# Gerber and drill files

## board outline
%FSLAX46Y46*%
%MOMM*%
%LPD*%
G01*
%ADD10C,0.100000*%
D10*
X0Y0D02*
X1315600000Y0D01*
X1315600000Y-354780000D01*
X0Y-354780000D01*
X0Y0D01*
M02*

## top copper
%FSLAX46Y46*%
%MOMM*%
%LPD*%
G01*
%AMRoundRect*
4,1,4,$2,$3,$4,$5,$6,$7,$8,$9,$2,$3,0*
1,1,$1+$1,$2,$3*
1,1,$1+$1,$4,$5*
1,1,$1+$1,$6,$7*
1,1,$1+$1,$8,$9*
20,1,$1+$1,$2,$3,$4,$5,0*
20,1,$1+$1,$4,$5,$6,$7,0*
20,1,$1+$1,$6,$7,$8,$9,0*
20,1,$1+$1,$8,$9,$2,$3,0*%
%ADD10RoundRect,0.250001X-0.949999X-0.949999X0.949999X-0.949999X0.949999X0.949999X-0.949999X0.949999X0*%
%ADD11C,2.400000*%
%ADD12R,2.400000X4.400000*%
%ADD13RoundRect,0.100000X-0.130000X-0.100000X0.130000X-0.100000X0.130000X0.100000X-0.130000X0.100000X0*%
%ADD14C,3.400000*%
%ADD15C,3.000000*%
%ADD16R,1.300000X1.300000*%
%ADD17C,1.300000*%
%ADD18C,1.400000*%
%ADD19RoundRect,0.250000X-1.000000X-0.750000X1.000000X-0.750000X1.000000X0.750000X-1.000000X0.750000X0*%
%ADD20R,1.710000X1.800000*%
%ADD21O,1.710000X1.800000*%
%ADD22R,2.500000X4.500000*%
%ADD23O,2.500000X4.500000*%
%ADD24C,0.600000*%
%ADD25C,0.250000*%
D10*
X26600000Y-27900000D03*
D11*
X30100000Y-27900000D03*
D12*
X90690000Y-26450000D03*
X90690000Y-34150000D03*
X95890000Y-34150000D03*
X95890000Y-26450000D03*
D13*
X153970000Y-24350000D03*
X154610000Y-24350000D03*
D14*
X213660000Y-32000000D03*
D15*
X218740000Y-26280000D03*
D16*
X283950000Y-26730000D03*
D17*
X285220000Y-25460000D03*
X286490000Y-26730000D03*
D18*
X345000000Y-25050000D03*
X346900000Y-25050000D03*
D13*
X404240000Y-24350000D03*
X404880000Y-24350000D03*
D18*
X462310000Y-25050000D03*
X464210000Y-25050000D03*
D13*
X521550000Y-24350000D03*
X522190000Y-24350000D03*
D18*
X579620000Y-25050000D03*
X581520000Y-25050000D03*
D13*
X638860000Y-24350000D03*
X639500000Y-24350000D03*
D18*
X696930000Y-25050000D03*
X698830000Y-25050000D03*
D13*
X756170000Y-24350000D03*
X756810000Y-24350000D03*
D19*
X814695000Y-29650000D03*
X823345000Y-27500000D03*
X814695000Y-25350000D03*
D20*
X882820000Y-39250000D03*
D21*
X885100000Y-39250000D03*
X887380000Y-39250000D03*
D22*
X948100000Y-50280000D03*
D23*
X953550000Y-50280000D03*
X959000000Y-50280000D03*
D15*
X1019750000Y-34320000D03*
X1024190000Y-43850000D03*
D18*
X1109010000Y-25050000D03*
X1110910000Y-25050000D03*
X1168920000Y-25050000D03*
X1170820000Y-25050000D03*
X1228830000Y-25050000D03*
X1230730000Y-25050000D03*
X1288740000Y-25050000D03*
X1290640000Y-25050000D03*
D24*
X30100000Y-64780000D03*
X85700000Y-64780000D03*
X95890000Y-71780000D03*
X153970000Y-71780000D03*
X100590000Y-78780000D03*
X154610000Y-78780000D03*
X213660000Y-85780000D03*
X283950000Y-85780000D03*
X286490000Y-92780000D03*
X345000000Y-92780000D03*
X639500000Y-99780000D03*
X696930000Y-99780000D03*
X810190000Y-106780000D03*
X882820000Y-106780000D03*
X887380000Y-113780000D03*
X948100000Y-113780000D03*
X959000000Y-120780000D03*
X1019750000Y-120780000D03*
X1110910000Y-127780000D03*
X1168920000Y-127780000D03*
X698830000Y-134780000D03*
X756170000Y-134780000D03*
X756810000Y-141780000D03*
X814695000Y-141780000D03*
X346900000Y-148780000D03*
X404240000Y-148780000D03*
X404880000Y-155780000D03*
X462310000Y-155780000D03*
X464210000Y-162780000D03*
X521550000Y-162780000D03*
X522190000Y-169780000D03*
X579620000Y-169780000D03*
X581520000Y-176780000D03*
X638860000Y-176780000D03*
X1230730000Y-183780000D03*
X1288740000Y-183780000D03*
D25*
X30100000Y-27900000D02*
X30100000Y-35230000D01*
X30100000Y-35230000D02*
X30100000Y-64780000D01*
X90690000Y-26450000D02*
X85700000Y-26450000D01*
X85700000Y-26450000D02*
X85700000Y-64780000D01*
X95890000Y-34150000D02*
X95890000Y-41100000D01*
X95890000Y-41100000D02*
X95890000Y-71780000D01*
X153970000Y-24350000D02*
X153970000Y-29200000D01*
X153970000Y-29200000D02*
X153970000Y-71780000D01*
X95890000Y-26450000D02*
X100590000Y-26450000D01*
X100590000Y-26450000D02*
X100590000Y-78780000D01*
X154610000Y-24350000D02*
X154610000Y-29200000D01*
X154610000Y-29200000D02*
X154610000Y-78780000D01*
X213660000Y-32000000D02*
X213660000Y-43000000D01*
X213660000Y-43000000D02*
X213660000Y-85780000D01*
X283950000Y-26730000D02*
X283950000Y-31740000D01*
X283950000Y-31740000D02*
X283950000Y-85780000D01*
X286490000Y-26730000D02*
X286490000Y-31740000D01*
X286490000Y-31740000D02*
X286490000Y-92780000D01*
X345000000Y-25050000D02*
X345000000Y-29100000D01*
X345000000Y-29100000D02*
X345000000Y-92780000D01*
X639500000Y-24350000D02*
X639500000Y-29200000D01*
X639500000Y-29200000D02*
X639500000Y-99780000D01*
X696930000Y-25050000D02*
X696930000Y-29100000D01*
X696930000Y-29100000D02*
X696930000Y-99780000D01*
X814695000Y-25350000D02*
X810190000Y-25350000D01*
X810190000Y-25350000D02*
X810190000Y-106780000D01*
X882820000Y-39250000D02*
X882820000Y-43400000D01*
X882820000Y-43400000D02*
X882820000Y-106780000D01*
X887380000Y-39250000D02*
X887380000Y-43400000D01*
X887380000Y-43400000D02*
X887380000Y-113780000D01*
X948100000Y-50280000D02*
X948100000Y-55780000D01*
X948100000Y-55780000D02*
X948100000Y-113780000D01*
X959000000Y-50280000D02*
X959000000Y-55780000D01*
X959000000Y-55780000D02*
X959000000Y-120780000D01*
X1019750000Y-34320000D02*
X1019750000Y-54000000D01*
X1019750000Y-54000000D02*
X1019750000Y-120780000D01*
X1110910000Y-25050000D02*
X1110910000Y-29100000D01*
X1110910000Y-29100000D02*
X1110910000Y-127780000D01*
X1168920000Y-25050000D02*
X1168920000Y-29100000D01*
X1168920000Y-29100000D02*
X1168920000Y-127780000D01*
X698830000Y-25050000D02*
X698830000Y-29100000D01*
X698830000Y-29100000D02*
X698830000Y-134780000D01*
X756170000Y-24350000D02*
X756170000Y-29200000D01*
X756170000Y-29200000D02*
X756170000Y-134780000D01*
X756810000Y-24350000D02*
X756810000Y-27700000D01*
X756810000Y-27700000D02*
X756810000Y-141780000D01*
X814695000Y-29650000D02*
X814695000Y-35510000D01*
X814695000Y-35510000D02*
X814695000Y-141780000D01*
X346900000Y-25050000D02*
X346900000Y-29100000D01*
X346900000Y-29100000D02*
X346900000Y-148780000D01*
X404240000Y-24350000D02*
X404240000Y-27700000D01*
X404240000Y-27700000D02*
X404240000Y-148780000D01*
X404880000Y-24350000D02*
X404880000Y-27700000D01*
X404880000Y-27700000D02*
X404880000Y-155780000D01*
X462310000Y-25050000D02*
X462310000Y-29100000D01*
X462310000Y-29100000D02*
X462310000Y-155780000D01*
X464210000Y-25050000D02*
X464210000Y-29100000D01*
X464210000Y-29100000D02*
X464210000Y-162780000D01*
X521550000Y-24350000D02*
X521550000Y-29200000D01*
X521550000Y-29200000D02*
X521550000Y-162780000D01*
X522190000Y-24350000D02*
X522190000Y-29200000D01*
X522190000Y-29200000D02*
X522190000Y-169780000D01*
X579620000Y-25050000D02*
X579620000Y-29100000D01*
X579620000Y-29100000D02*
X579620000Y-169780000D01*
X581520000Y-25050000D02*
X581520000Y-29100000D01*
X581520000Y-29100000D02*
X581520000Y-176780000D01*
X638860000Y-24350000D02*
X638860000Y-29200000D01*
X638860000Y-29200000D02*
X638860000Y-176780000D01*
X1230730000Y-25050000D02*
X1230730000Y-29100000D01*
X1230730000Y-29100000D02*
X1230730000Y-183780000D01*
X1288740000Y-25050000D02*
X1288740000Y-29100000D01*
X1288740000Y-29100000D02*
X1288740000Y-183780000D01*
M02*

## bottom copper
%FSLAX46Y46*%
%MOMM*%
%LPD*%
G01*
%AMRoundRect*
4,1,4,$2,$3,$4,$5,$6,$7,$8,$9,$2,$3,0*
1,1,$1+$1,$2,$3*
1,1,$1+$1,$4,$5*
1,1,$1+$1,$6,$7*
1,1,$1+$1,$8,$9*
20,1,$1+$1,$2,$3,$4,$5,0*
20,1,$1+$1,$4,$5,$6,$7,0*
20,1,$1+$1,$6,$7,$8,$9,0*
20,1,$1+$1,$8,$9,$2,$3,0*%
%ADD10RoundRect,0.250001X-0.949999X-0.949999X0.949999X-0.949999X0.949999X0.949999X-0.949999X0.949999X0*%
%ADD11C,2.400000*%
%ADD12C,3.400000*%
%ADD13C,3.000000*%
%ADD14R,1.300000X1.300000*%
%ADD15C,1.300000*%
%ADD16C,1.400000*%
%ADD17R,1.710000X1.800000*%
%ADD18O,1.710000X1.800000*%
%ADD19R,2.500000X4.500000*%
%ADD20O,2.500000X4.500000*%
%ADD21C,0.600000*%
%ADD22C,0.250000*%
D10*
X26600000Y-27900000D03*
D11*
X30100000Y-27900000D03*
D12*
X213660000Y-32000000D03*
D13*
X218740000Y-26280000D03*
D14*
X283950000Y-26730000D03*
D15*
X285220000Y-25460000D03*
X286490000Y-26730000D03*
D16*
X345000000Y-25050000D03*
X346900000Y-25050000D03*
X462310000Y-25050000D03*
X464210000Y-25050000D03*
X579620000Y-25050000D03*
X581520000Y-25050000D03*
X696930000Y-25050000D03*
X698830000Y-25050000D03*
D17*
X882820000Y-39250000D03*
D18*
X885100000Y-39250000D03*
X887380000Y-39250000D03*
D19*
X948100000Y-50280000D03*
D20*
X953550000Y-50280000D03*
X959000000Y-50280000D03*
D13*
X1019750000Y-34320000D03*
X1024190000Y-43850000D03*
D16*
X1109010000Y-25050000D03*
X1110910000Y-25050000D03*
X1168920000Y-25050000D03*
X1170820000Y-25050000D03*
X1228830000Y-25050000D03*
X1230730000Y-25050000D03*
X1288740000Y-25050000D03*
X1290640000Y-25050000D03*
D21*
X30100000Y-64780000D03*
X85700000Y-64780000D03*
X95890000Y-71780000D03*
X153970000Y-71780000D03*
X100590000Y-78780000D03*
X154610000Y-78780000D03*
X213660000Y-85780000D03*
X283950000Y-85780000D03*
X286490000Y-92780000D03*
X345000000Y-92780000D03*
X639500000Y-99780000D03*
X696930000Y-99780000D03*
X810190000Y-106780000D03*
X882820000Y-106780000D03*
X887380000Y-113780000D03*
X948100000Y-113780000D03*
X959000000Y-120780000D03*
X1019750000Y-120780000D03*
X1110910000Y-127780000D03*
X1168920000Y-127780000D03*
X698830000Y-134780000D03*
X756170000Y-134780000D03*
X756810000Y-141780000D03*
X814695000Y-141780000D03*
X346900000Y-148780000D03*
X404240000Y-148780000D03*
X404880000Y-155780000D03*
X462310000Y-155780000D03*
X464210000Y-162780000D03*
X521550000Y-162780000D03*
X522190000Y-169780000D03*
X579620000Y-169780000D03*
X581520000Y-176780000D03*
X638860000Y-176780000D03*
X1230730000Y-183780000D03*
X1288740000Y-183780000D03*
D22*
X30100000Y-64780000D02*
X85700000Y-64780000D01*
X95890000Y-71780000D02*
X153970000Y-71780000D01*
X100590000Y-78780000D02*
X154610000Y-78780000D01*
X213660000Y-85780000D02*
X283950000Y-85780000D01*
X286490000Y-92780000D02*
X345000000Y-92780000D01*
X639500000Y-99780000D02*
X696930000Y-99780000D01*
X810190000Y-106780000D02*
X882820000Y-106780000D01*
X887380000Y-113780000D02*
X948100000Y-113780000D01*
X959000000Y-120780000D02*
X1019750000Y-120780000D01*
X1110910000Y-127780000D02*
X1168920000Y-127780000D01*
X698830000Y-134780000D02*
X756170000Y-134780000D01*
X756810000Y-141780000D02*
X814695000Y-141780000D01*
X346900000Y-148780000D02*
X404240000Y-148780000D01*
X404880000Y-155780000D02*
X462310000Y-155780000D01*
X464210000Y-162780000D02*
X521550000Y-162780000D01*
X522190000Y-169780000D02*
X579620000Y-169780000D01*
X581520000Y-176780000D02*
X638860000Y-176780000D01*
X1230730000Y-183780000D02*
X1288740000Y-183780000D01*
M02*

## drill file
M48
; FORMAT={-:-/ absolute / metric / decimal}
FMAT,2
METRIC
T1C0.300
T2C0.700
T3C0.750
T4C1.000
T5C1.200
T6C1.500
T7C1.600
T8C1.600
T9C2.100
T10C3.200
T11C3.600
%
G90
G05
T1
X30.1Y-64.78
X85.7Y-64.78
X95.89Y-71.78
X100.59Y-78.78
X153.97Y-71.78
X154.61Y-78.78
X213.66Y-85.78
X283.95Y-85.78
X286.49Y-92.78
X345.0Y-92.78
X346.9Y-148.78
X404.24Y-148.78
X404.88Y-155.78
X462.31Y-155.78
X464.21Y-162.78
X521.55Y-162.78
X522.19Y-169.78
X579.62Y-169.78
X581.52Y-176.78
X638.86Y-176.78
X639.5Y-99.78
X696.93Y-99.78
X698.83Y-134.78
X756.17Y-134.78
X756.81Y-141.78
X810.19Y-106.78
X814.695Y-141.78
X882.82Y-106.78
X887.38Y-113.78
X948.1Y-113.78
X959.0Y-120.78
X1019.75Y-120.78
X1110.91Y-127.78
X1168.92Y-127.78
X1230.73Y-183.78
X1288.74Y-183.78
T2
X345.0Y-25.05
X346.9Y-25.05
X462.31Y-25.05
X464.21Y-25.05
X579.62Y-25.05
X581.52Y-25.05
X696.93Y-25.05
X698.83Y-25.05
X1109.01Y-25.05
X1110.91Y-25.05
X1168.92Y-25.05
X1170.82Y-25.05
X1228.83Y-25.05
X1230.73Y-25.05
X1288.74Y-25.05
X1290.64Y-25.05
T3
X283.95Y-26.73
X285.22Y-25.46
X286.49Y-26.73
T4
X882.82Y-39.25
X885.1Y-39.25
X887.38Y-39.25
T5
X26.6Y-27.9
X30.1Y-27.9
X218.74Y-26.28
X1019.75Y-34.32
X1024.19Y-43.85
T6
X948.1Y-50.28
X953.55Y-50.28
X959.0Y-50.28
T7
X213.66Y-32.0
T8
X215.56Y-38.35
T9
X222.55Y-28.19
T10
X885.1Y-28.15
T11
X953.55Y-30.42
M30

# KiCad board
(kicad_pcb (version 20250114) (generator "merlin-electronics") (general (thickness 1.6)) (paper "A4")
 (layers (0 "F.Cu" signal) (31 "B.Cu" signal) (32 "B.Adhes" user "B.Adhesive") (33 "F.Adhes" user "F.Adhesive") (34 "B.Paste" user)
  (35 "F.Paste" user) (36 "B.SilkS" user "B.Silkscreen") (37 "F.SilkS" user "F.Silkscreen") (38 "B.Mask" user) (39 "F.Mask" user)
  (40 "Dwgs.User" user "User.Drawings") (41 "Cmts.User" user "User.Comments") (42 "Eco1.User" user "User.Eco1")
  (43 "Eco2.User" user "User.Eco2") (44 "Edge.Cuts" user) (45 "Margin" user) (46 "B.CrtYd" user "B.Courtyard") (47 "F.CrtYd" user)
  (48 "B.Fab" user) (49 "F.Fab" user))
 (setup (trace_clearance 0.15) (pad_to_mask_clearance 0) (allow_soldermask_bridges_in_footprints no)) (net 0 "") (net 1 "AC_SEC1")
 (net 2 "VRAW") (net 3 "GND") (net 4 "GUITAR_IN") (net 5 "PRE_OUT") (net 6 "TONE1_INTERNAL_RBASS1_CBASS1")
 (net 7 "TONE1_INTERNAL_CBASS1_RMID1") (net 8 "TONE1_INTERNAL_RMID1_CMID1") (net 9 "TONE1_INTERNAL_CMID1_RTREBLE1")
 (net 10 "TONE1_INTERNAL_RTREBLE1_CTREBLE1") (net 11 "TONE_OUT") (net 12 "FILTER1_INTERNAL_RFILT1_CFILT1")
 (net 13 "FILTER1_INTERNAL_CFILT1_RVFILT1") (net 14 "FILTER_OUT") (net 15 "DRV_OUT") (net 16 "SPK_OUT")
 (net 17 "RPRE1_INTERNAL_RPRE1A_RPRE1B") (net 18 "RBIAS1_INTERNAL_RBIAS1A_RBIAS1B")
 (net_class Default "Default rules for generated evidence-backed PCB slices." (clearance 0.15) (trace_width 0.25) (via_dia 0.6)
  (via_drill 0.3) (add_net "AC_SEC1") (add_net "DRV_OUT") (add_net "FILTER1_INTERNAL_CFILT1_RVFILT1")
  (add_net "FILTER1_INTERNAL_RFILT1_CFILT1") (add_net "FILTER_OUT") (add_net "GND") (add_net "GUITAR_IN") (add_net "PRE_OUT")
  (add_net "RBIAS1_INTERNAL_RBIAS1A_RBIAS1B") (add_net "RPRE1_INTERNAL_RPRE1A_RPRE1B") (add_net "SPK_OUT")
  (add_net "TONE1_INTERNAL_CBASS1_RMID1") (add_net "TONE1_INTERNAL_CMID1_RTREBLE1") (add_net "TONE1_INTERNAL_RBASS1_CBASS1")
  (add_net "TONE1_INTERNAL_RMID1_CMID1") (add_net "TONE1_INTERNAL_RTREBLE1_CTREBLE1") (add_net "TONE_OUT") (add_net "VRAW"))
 (gr_rect (start 0 0) (end 1315.6 354.78) (stroke (width 0.1) (type default)) (fill no) (layer "Edge.Cuts"))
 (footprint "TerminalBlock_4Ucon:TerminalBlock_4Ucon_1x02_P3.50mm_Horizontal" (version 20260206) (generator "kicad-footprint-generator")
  (layer "F.Cu") (at 26.6 27.9 0)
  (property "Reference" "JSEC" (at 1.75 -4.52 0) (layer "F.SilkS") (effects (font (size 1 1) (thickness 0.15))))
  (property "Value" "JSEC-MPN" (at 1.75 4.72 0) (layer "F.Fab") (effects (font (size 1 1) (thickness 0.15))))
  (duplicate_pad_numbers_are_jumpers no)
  (pad "1" thru_hole roundrect (at 0 0) (size 2.4 2.4) (drill 1.2) (layers "*.Cu" "*.Mask") (remove_unused_layers no)
   (roundrect_rratio 0.104167))
  (pad "2" thru_hole circle (at 3.5 0) (size 2.4 2.4) (drill 1.2) (layers "*.Cu" "*.Mask") (remove_unused_layers no) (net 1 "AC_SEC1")))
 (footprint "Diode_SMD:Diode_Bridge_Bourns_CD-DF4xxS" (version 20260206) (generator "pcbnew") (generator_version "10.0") (layer "F.Cu")
  (at 93.29 30.3 0)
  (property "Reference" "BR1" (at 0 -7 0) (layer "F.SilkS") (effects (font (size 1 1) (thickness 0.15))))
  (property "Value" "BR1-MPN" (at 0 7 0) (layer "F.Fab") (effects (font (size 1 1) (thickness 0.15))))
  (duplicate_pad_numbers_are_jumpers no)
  (pad "1" smd rect (at -2.6 -3.85) (size 2.4 4.4) (layers "F.Cu" "F.Mask" "F.Paste") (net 1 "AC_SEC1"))
  (pad "2" smd rect (at -2.6 3.85) (size 2.4 4.4) (layers "F.Cu" "F.Mask" "F.Paste"))
  (pad "3" smd rect (at 2.6 3.85) (size 2.4 4.4) (layers "F.Cu" "F.Mask" "F.Paste") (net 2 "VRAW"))
  (pad "4" smd rect (at 2.6 -3.85) (size 2.4 4.4) (layers "F.Cu" "F.Mask" "F.Paste") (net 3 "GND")))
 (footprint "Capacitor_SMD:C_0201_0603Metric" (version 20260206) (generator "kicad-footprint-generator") (layer "F.Cu") (at 154.29 24.35 0)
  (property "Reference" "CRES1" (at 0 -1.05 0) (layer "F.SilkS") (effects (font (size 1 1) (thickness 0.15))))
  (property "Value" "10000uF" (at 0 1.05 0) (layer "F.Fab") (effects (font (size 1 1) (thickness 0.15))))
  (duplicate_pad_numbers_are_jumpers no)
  (pad "" smd roundrect (at -0.345 0) (size 0.318 0.36) (layers "F.Paste") (roundrect_rratio 0.25))
  (pad "" smd roundrect (at 0.345 0) (size 0.318 0.36) (layers "F.Paste") (roundrect_rratio 0.25))
  (pad "1" smd roundrect (at -0.32 0) (size 0.46 0.4) (layers "F.Cu" "F.Mask") (roundrect_rratio 0.25) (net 2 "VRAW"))
  (pad "2" smd roundrect (at 0.32 0) (size 0.46 0.4) (layers "F.Cu" "F.Mask") (roundrect_rratio 0.25) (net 3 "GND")))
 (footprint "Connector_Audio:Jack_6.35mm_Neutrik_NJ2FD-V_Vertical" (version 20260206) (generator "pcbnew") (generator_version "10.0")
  (layer "F.Cu") (at 218.74 26.28 0)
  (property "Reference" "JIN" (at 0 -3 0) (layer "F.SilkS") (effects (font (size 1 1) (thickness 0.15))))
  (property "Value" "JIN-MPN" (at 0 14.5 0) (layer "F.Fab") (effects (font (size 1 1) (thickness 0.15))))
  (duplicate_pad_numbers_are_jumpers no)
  (pad "" np_thru_hole circle (at -3.18 12.07 180) (size 1.6 1.6) (drill 1.6) (layers "*.Cu" "*.Mask"))
  (pad "" np_thru_hole circle (at 3.81 1.91 180) (size 2.1 2.1) (drill 2.1) (layers "*.Cu" "*.Mask"))
  (pad "S" thru_hole circle (at -5.08 5.72 180) (size 3.4 3.4) (drill 1.6) (layers "*.Cu" "*.Mask") (remove_unused_layers no)
   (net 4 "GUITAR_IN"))
  (pad "T" thru_hole circle (at 0 0 180) (size 3 3) (drill 1.2) (layers "*.Cu" "*.Mask") (remove_unused_layers no)))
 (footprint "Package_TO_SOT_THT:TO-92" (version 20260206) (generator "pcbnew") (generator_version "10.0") (layer "F.Cu") (at 283.95 26.73 0)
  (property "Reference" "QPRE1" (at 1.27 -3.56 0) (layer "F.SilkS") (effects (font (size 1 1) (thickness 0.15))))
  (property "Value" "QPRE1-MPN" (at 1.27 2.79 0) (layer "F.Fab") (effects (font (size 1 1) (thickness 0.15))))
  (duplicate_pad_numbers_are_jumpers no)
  (pad "1" thru_hole rect (at 0 0) (size 1.3 1.3) (drill 0.75) (layers "*.Cu" "*.Mask") (remove_unused_layers no) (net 4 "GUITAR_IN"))
  (pad "2" thru_hole circle (at 1.27 -1.27) (size 1.3 1.3) (drill 0.75) (layers "*.Cu" "*.Mask") (remove_unused_layers no))
  (pad "3" thru_hole circle (at 2.54 0) (size 1.3 1.3) (drill 0.75) (layers "*.Cu" "*.Mask") (remove_unused_layers no) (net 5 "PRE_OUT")))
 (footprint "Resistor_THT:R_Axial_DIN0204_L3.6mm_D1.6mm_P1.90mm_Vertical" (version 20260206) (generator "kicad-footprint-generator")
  (layer "F.Cu") (at 345 25.05 0)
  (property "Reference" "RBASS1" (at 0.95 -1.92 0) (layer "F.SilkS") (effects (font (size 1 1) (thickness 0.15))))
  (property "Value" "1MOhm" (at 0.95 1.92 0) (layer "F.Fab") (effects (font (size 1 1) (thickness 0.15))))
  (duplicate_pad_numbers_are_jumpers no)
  (pad "1" thru_hole circle (at 0 0) (size 1.4 1.4) (drill 0.7) (layers "*.Cu" "*.Mask") (remove_unused_layers no) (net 5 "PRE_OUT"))
  (pad "2" thru_hole circle (at 1.9 0) (size 1.4 1.4) (drill 0.7) (layers "*.Cu" "*.Mask") (remove_unused_layers no)
   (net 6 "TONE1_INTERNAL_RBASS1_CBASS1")))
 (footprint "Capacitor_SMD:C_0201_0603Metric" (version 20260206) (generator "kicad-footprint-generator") (layer "F.Cu") (at 404.56 24.35 0)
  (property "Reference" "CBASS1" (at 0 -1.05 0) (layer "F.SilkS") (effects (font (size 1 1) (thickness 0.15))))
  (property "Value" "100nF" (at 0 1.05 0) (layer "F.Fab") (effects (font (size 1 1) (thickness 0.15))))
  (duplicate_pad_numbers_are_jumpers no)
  (pad "" smd roundrect (at -0.345 0) (size 0.318 0.36) (layers "F.Paste") (roundrect_rratio 0.25))
  (pad "" smd roundrect (at 0.345 0) (size 0.318 0.36) (layers "F.Paste") (roundrect_rratio 0.25))
  (pad "1" smd roundrect (at -0.32 0) (size 0.46 0.4) (layers "F.Cu" "F.Mask") (roundrect_rratio 0.25)
   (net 6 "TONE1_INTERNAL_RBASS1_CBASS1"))
  (pad "2" smd roundrect (at 0.32 0) (size 0.46 0.4) (layers "F.Cu" "F.Mask") (roundrect_rratio 0.25) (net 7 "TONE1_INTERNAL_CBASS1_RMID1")))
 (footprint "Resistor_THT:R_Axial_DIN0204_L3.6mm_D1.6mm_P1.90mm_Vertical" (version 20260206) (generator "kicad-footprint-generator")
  (layer "F.Cu") (at 462.31 25.05 0)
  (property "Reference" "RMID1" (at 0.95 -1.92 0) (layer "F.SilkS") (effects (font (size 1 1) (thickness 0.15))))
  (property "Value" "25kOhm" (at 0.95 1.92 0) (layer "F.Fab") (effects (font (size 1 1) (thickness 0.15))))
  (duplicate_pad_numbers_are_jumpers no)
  (pad "1" thru_hole circle (at 0 0) (size 1.4 1.4) (drill 0.7) (layers "*.Cu" "*.Mask") (remove_unused_layers no)
   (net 7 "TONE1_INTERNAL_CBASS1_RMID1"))
  (pad "2" thru_hole circle (at 1.9 0) (size 1.4 1.4) (drill 0.7) (layers "*.Cu" "*.Mask") (remove_unused_layers no)
   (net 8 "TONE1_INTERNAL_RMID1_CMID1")))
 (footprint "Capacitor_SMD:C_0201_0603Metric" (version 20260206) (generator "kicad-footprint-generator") (layer "F.Cu") (at 521.87 24.35 0)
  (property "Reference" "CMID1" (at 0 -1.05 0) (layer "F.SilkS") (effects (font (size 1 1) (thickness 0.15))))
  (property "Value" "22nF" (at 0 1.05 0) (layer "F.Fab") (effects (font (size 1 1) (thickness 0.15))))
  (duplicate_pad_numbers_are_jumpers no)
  (pad "" smd roundrect (at -0.345 0) (size 0.318 0.36) (layers "F.Paste") (roundrect_rratio 0.25))
  (pad "" smd roundrect (at 0.345 0) (size 0.318 0.36) (layers "F.Paste") (roundrect_rratio 0.25))
  (pad "1" smd roundrect (at -0.32 0) (size 0.46 0.4) (layers "F.Cu" "F.Mask") (roundrect_rratio 0.25) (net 8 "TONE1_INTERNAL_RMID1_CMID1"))
  (pad "2" smd roundrect (at 0.32 0) (size 0.46 0.4) (layers "F.Cu" "F.Mask") (roundrect_rratio 0.25)
   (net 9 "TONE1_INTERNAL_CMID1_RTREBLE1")))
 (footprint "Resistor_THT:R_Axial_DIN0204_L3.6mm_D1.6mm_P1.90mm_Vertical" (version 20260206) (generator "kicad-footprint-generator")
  (layer "F.Cu") (at 579.62 25.05 0)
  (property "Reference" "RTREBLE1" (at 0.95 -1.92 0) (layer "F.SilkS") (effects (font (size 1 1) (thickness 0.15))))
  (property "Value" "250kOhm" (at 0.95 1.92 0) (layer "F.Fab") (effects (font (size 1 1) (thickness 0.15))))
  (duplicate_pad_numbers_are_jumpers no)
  (pad "1" thru_hole circle (at 0 0) (size 1.4 1.4) (drill 0.7) (layers "*.Cu" "*.Mask") (remove_unused_layers no)
   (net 9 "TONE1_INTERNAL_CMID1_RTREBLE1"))
  (pad "2" thru_hole circle (at 1.9 0) (size 1.4 1.4) (drill 0.7) (layers "*.Cu" "*.Mask") (remove_unused_layers no)
   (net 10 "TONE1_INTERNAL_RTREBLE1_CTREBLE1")))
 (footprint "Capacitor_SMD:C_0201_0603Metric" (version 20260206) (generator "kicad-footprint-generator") (layer "F.Cu") (at 639.18 24.35 0)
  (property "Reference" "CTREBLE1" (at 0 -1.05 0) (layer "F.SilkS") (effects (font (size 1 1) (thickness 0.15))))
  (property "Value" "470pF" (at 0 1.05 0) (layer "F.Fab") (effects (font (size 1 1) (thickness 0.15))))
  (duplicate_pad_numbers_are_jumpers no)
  (pad "" smd roundrect (at -0.345 0) (size 0.318 0.36) (layers "F.Paste") (roundrect_rratio 0.25))
  (pad "" smd roundrect (at 0.345 0) (size 0.318 0.36) (layers "F.Paste") (roundrect_rratio 0.25))
  (pad "1" smd roundrect (at -0.32 0) (size 0.46 0.4) (layers "F.Cu" "F.Mask") (roundrect_rratio 0.25)
   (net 10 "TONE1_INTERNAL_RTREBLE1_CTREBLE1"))
  (pad "2" smd roundrect (at 0.32 0) (size 0.46 0.4) (layers "F.Cu" "F.Mask") (roundrect_rratio 0.25) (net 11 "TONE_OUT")))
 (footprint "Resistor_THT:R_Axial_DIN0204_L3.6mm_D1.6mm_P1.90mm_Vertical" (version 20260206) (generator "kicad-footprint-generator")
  (layer "F.Cu") (at 696.93 25.05 0)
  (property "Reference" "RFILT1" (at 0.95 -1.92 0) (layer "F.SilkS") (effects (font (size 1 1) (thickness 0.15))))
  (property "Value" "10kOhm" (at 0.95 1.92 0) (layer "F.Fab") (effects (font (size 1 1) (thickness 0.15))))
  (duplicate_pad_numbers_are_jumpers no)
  (pad "1" thru_hole circle (at 0 0) (size 1.4 1.4) (drill 0.7) (layers "*.Cu" "*.Mask") (remove_unused_layers no) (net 11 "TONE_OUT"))
  (pad "2" thru_hole circle (at 1.9 0) (size 1.4 1.4) (drill 0.7) (layers "*.Cu" "*.Mask") (remove_unused_layers no)
   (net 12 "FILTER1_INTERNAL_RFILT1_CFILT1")))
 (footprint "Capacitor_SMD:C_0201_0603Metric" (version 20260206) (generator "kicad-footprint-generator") (layer "F.Cu") (at 756.49 24.35 0)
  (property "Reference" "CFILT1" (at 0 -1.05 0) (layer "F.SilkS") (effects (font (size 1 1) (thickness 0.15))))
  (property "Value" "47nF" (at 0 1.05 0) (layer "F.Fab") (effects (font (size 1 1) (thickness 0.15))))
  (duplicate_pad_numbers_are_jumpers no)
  (pad "" smd roundrect (at -0.345 0) (size 0.318 0.36) (layers "F.Paste") (roundrect_rratio 0.25))
  (pad "" smd roundrect (at 0.345 0) (size 0.318 0.36) (layers "F.Paste") (roundrect_rratio 0.25))
  (pad "1" smd roundrect (at -0.32 0) (size 0.46 0.4) (layers "F.Cu" "F.Mask") (roundrect_rratio 0.25)
   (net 12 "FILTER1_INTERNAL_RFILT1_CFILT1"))
  (pad "2" smd roundrect (at 0.32 0) (size 0.46 0.4) (layers "F.Cu" "F.Mask") (roundrect_rratio 0.25)
   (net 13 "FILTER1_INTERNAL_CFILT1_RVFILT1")))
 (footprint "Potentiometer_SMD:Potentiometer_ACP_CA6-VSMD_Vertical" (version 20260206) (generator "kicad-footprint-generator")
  (layer "F.Cu") (at 819.02 27.5 0)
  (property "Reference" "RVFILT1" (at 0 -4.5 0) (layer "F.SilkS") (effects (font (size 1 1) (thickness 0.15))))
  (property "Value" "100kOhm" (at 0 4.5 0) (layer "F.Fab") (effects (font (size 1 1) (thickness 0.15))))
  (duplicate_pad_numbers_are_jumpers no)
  (pad "1" smd roundrect (at -4.325 2.15) (size 2.5 2) (layers "F.Cu" "F.Mask" "F.Paste") (roundrect_rratio 0.125)
   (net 13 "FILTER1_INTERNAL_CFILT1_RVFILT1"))
  (pad "2" smd roundrect (at 4.325 0) (size 2.5 2) (layers "F.Cu" "F.Mask" "F.Paste") (roundrect_rratio 0.125))
  (pad "3" smd roundrect (at -4.325 -2.15) (size 2.5 2) (layers "F.Cu" "F.Mask" "F.Paste") (roundrect_rratio 0.125) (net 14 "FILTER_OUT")))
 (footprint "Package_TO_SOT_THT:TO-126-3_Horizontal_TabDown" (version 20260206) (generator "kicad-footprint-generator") (layer "F.Cu")
  (at 882.82 39.25 0)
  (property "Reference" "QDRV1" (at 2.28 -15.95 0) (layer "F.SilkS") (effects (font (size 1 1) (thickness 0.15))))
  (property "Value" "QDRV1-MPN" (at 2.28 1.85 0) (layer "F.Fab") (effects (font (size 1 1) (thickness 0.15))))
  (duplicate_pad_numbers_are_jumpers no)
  (pad "" np_thru_hole circle (at 2.28 -11.1) (size 3.2 3.2) (drill 3.2) (layers "*.Cu" "*.Mask"))
  (pad "1" thru_hole rect (at 0 0) (size 1.71 1.8) (drill 1) (layers "*.Cu" "*.Mask") (remove_unused_layers no) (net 14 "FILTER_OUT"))
  (pad "2" thru_hole oval (at 2.28 0) (size 1.71 1.8) (drill 1) (layers "*.Cu" "*.Mask") (remove_unused_layers no))
  (pad "3" thru_hole oval (at 4.56 0) (size 1.71 1.8) (drill 1) (layers "*.Cu" "*.Mask") (remove_unused_layers no) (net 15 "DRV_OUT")))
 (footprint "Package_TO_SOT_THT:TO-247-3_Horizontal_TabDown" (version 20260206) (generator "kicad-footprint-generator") (layer "F.Cu")
  (at 948.1 50.28 0)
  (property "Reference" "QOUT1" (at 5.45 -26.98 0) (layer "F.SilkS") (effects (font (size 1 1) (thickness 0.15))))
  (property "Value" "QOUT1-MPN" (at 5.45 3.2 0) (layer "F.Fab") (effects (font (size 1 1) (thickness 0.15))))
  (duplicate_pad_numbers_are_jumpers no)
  (pad "" np_thru_hole circle (at 5.45 -19.86) (size 3.6 3.6) (drill 3.6) (layers "*.Cu" "*.Mask"))
  (pad "1" thru_hole rect (at 0 0) (size 2.5 4.5) (drill 1.5) (layers "*.Cu" "*.Mask") (remove_unused_layers no) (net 15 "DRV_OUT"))
  (pad "2" thru_hole oval (at 5.45 0) (size 2.5 4.5) (drill 1.5) (layers "*.Cu" "*.Mask") (remove_unused_layers no))
  (pad "3" thru_hole oval (at 10.9 0) (size 2.5 4.5) (drill 1.5) (layers "*.Cu" "*.Mask") (remove_unused_layers no) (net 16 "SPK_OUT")))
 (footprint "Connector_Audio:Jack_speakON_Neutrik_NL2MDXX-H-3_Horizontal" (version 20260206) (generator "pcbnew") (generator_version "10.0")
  (layer "F.Cu") (at 1019.75 34.32 0)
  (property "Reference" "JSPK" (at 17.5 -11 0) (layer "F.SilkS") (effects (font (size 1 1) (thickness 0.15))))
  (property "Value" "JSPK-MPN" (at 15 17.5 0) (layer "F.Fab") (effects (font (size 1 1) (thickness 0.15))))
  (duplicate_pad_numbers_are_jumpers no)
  (pad "1+" thru_hole circle (at 0 0) (size 3 3) (drill 1.2) (layers "*.Cu" "*.Mask") (remove_unused_layers no) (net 16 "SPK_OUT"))
  (pad "1-" thru_hole circle (at 4.44 9.53) (size 3 3) (drill 1.2) (layers "*.Cu" "*.Mask") (remove_unused_layers no)))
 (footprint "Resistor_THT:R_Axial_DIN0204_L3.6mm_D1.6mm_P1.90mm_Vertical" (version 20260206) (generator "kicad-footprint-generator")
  (layer "F.Cu") (at 1109.01 25.05 0)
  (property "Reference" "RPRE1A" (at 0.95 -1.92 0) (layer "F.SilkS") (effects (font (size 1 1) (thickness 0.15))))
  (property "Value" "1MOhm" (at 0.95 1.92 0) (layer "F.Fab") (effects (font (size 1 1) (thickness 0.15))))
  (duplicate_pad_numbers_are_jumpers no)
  (pad "1" thru_hole circle (at 0 0) (size 1.4 1.4) (drill 0.7) (layers "*.Cu" "*.Mask") (remove_unused_layers no))
  (pad "2" thru_hole circle (at 1.9 0) (size 1.4 1.4) (drill 0.7) (layers "*.Cu" "*.Mask") (remove_unused_layers no)
   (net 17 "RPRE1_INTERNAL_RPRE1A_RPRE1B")))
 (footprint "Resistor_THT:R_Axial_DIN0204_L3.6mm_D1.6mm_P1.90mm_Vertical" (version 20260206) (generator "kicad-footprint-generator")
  (layer "F.Cu") (at 1168.92 25.05 0)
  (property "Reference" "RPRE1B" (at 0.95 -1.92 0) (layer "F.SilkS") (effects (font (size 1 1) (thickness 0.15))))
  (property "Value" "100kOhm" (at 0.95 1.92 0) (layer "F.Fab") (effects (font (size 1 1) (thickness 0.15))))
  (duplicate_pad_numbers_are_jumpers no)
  (pad "1" thru_hole circle (at 0 0) (size 1.4 1.4) (drill 0.7) (layers "*.Cu" "*.Mask") (remove_unused_layers no)
   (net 17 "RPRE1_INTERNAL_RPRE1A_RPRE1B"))
  (pad "2" thru_hole circle (at 1.9 0) (size 1.4 1.4) (drill 0.7) (layers "*.Cu" "*.Mask") (remove_unused_layers no)))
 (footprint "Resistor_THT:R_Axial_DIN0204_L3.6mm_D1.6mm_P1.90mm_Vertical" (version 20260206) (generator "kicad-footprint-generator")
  (layer "F.Cu") (at 1228.83 25.05 0)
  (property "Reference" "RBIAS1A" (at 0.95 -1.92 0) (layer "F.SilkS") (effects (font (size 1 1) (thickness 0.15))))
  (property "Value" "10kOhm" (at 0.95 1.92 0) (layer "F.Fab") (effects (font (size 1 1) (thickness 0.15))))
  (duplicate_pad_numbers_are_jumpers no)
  (pad "1" thru_hole circle (at 0 0) (size 1.4 1.4) (drill 0.7) (layers "*.Cu" "*.Mask") (remove_unused_layers no))
  (pad "2" thru_hole circle (at 1.9 0) (size 1.4 1.4) (drill 0.7) (layers "*.Cu" "*.Mask") (remove_unused_layers no)
   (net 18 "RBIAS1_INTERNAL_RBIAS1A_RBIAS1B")))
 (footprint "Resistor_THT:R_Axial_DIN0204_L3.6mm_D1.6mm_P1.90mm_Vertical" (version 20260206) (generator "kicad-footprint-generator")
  (layer "F.Cu") (at 1288.74 25.05 0)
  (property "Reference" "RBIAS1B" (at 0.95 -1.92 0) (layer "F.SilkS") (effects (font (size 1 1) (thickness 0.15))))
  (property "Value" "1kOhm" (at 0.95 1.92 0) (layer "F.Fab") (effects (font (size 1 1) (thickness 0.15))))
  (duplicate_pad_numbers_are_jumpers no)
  (pad "1" thru_hole circle (at 0 0) (size 1.4 1.4) (drill 0.7) (layers "*.Cu" "*.Mask") (remove_unused_layers no)
   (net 18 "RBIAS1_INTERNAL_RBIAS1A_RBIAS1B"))
  (pad "2" thru_hole circle (at 1.9 0) (size 1.4 1.4) (drill 0.7) (layers "*.Cu" "*.Mask") (remove_unused_layers no)))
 (segment (start 30.1 27.9) (end 30.1 35.23) (width 0.25) (layer "F.Cu") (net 1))
 (segment (start 30.1 35.23) (end 30.1 64.78) (width 0.25) (layer "F.Cu") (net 1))
 (via (at 30.1 64.78) (size 0.6) (drill 0.3) (layers "F.Cu" "B.Cu") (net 1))
 (segment (start 90.69 26.45) (end 85.7 26.45) (width 0.25) (layer "F.Cu") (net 1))
 (segment (start 85.7 26.45) (end 85.7 64.78) (width 0.25) (layer "F.Cu") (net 1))
 (via (at 85.7 64.78) (size 0.6) (drill 0.3) (layers "F.Cu" "B.Cu") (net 1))
 (segment (start 30.1 64.78) (end 85.7 64.78) (width 0.25) (layer "B.Cu") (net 1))
 (segment (start 95.89 34.15) (end 95.89 41.1) (width 0.25) (layer "F.Cu") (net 2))
 (segment (start 95.89 41.1) (end 95.89 71.78) (width 0.25) (layer "F.Cu") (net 2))
 (via (at 95.89 71.78) (size 0.6) (drill 0.3) (layers "F.Cu" "B.Cu") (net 2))
 (segment (start 153.97 24.35) (end 153.97 29.2) (width 0.25) (layer "F.Cu") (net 2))
 (segment (start 153.97 29.2) (end 153.97 71.78) (width 0.25) (layer "F.Cu") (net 2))
 (via (at 153.97 71.78) (size 0.6) (drill 0.3) (layers "F.Cu" "B.Cu") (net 2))
 (segment (start 95.89 71.78) (end 153.97 71.78) (width 0.25) (layer "B.Cu") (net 2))
 (segment (start 95.89 26.45) (end 100.59 26.45) (width 0.25) (layer "F.Cu") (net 3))
 (segment (start 100.59 26.45) (end 100.59 78.78) (width 0.25) (layer "F.Cu") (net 3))
 (via (at 100.59 78.78) (size 0.6) (drill 0.3) (layers "F.Cu" "B.Cu") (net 3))
 (segment (start 154.61 24.35) (end 154.61 29.2) (width 0.25) (layer "F.Cu") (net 3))
 (segment (start 154.61 29.2) (end 154.61 78.78) (width 0.25) (layer "F.Cu") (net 3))
 (via (at 154.61 78.78) (size 0.6) (drill 0.3) (layers "F.Cu" "B.Cu") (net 3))
 (segment (start 100.59 78.78) (end 154.61 78.78) (width 0.25) (layer "B.Cu") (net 3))
 (segment (start 213.66 32) (end 213.66 43) (width 0.25) (layer "F.Cu") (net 4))
 (segment (start 213.66 43) (end 213.66 85.78) (width 0.25) (layer "F.Cu") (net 4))
 (via (at 213.66 85.78) (size 0.6) (drill 0.3) (layers "F.Cu" "B.Cu") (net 4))
 (segment (start 283.95 26.73) (end 283.95 31.74) (width 0.25) (layer "F.Cu") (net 4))
 (segment (start 283.95 31.74) (end 283.95 85.78) (width 0.25) (layer "F.Cu") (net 4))
 (via (at 283.95 85.78) (size 0.6) (drill 0.3) (layers "F.Cu" "B.Cu") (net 4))
 (segment (start 213.66 85.78) (end 283.95 85.78) (width 0.25) (layer "B.Cu") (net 4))
 (segment (start 286.49 26.73) (end 286.49 31.74) (width 0.25) (layer "F.Cu") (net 5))
 (segment (start 286.49 31.74) (end 286.49 92.78) (width 0.25) (layer "F.Cu") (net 5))
 (via (at 286.49 92.78) (size 0.6) (drill 0.3) (layers "F.Cu" "B.Cu") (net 5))
 (segment (start 345 25.05) (end 345 29.1) (width 0.25) (layer "F.Cu") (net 5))
 (segment (start 345 29.1) (end 345 92.78) (width 0.25) (layer "F.Cu") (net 5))
 (via (at 345 92.78) (size 0.6) (drill 0.3) (layers "F.Cu" "B.Cu") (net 5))
 (segment (start 286.49 92.78) (end 345 92.78) (width 0.25) (layer "B.Cu") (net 5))
 (segment (start 639.5 24.35) (end 639.5 29.2) (width 0.25) (layer "F.Cu") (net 11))
 (segment (start 639.5 29.2) (end 639.5 99.78) (width 0.25) (layer "F.Cu") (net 11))
 (via (at 639.5 99.78) (size 0.6) (drill 0.3) (layers "F.Cu" "B.Cu") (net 11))
 (segment (start 696.93 25.05) (end 696.93 29.1) (width 0.25) (layer "F.Cu") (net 11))
 (segment (start 696.93 29.1) (end 696.93 99.78) (width 0.25) (layer "F.Cu") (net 11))
 (via (at 696.93 99.78) (size 0.6) (drill 0.3) (layers "F.Cu" "B.Cu") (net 11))
 (segment (start 639.5 99.78) (end 696.93 99.78) (width 0.25) (layer "B.Cu") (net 11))
 (segment (start 814.695 25.35) (end 810.19 25.35) (width 0.25) (layer "F.Cu") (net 14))
 (segment (start 810.19 25.35) (end 810.19 106.78) (width 0.25) (layer "F.Cu") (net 14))
 (via (at 810.19 106.78) (size 0.6) (drill 0.3) (layers "F.Cu" "B.Cu") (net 14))
 (segment (start 882.82 39.25) (end 882.82 43.4) (width 0.25) (layer "F.Cu") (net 14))
 (segment (start 882.82 43.4) (end 882.82 106.78) (width 0.25) (layer "F.Cu") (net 14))
 (via (at 882.82 106.78) (size 0.6) (drill 0.3) (layers "F.Cu" "B.Cu") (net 14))
 (segment (start 810.19 106.78) (end 882.82 106.78) (width 0.25) (layer "B.Cu") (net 14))
 (segment (start 887.38 39.25) (end 887.38 43.4) (width 0.25) (layer "F.Cu") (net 15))
 (segment (start 887.38 43.4) (end 887.38 113.78) (width 0.25) (layer "F.Cu") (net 15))
 (via (at 887.38 113.78) (size 0.6) (drill 0.3) (layers "F.Cu" "B.Cu") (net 15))
 (segment (start 948.1 50.28) (end 948.1 55.78) (width 0.25) (layer "F.Cu") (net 15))
 (segment (start 948.1 55.78) (end 948.1 113.78) (width 0.25) (layer "F.Cu") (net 15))
 (via (at 948.1 113.78) (size 0.6) (drill 0.3) (layers "F.Cu" "B.Cu") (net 15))
 (segment (start 887.38 113.78) (end 948.1 113.78) (width 0.25) (layer "B.Cu") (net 15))
 (segment (start 959 50.28) (end 959 55.78) (width 0.25) (layer "F.Cu") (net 16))
 (segment (start 959 55.78) (end 959 120.78) (width 0.25) (layer "F.Cu") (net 16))
 (via (at 959 120.78) (size 0.6) (drill 0.3) (layers "F.Cu" "B.Cu") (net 16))
 (segment (start 1019.75 34.32) (end 1019.75 54) (width 0.25) (layer "F.Cu") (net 16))
 (segment (start 1019.75 54) (end 1019.75 120.78) (width 0.25) (layer "F.Cu") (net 16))
 (via (at 1019.75 120.78) (size 0.6) (drill 0.3) (layers "F.Cu" "B.Cu") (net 16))
 (segment (start 959 120.78) (end 1019.75 120.78) (width 0.25) (layer "B.Cu") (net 16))
 (segment (start 1110.91 25.05) (end 1110.91 29.1) (width 0.25) (layer "F.Cu") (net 17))
 (segment (start 1110.91 29.1) (end 1110.91 127.78) (width 0.25) (layer "F.Cu") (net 17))
 (via (at 1110.91 127.78) (size 0.6) (drill 0.3) (layers "F.Cu" "B.Cu") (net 17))
 (segment (start 1168.92 25.05) (end 1168.92 29.1) (width 0.25) (layer "F.Cu") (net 17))
 (segment (start 1168.92 29.1) (end 1168.92 127.78) (width 0.25) (layer "F.Cu") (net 17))
 (via (at 1168.92 127.78) (size 0.6) (drill 0.3) (layers "F.Cu" "B.Cu") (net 17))
 (segment (start 1110.91 127.78) (end 1168.92 127.78) (width 0.25) (layer "B.Cu") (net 17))
 (segment (start 698.83 25.05) (end 698.83 29.1) (width 0.25) (layer "F.Cu") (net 12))
 (segment (start 698.83 29.1) (end 698.83 134.78) (width 0.25) (layer "F.Cu") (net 12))
 (via (at 698.83 134.78) (size 0.6) (drill 0.3) (layers "F.Cu" "B.Cu") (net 12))
 (segment (start 756.17 24.35) (end 756.17 29.2) (width 0.25) (layer "F.Cu") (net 12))
 (segment (start 756.17 29.2) (end 756.17 134.78) (width 0.25) (layer "F.Cu") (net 12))
 (via (at 756.17 134.78) (size 0.6) (drill 0.3) (layers "F.Cu" "B.Cu") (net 12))
 (segment (start 698.83 134.78) (end 756.17 134.78) (width 0.25) (layer "B.Cu") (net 12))
 (segment (start 756.81 24.35) (end 756.81 27.7) (width 0.25) (layer "F.Cu") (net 13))
 (segment (start 756.81 27.7) (end 756.81 141.78) (width 0.25) (layer "F.Cu") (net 13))
 (via (at 756.81 141.78) (size 0.6) (drill 0.3) (layers "F.Cu" "B.Cu") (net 13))
 (segment (start 814.695 29.65) (end 814.695 35.51) (width 0.25) (layer "F.Cu") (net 13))
 (segment (start 814.695 35.51) (end 814.695 141.78) (width 0.25) (layer "F.Cu") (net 13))
 (via (at 814.695 141.78) (size 0.6) (drill 0.3) (layers "F.Cu" "B.Cu") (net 13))
 (segment (start 756.81 141.78) (end 814.695 141.78) (width 0.25) (layer "B.Cu") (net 13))
 (segment (start 346.9 25.05) (end 346.9 29.1) (width 0.25) (layer "F.Cu") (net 6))
 (segment (start 346.9 29.1) (end 346.9 148.78) (width 0.25) (layer "F.Cu") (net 6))
 (via (at 346.9 148.78) (size 0.6) (drill 0.3) (layers "F.Cu" "B.Cu") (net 6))
 (segment (start 404.24 24.35) (end 404.24 27.7) (width 0.25) (layer "F.Cu") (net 6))
 (segment (start 404.24 27.7) (end 404.24 148.78) (width 0.25) (layer "F.Cu") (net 6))
 (via (at 404.24 148.78) (size 0.6) (drill 0.3) (layers "F.Cu" "B.Cu") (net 6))
 (segment (start 346.9 148.78) (end 404.24 148.78) (width 0.25) (layer "B.Cu") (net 6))
 (segment (start 404.88 24.35) (end 404.88 27.7) (width 0.25) (layer "F.Cu") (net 7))
 (segment (start 404.88 27.7) (end 404.88 155.78) (width 0.25) (layer "F.Cu") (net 7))
 (via (at 404.88 155.78) (size 0.6) (drill 0.3) (layers "F.Cu" "B.Cu") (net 7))
 (segment (start 462.31 25.05) (end 462.31 29.1) (width 0.25) (layer "F.Cu") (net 7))
 (segment (start 462.31 29.1) (end 462.31 155.78) (width 0.25) (layer "F.Cu") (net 7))
 (via (at 462.31 155.78) (size 0.6) (drill 0.3) (layers "F.Cu" "B.Cu") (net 7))
 (segment (start 404.88 155.78) (end 462.31 155.78) (width 0.25) (layer "B.Cu") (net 7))
 (segment (start 464.21 25.05) (end 464.21 29.1) (width 0.25) (layer "F.Cu") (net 8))
 (segment (start 464.21 29.1) (end 464.21 162.78) (width 0.25) (layer "F.Cu") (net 8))
 (via (at 464.21 162.78) (size 0.6) (drill 0.3) (layers "F.Cu" "B.Cu") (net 8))
 (segment (start 521.55 24.35) (end 521.55 29.2) (width 0.25) (layer "F.Cu") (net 8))
 (segment (start 521.55 29.2) (end 521.55 162.78) (width 0.25) (layer "F.Cu") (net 8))
 (via (at 521.55 162.78) (size 0.6) (drill 0.3) (layers "F.Cu" "B.Cu") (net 8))
 (segment (start 464.21 162.78) (end 521.55 162.78) (width 0.25) (layer "B.Cu") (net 8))
 (segment (start 522.19 24.35) (end 522.19 29.2) (width 0.25) (layer "F.Cu") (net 9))
 (segment (start 522.19 29.2) (end 522.19 169.78) (width 0.25) (layer "F.Cu") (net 9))
 (via (at 522.19 169.78) (size 0.6) (drill 0.3) (layers "F.Cu" "B.Cu") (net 9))
 (segment (start 579.62 25.05) (end 579.62 29.1) (width 0.25) (layer "F.Cu") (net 9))
 (segment (start 579.62 29.1) (end 579.62 169.78) (width 0.25) (layer "F.Cu") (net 9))
 (via (at 579.62 169.78) (size 0.6) (drill 0.3) (layers "F.Cu" "B.Cu") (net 9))
 (segment (start 522.19 169.78) (end 579.62 169.78) (width 0.25) (layer "B.Cu") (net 9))
 (segment (start 581.52 25.05) (end 581.52 29.1) (width 0.25) (layer "F.Cu") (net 10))
 (segment (start 581.52 29.1) (end 581.52 176.78) (width 0.25) (layer "F.Cu") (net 10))
 (via (at 581.52 176.78) (size 0.6) (drill 0.3) (layers "F.Cu" "B.Cu") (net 10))
 (segment (start 638.86 24.35) (end 638.86 29.2) (width 0.25) (layer "F.Cu") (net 10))
 (segment (start 638.86 29.2) (end 638.86 176.78) (width 0.25) (layer "F.Cu") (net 10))
 (via (at 638.86 176.78) (size 0.6) (drill 0.3) (layers "F.Cu" "B.Cu") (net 10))
 (segment (start 581.52 176.78) (end 638.86 176.78) (width 0.25) (layer "B.Cu") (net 10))
 (segment (start 1230.73 25.05) (end 1230.73 29.1) (width 0.25) (layer "F.Cu") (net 18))
 (segment (start 1230.73 29.1) (end 1230.73 183.78) (width 0.25) (layer "F.Cu") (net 18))
 (via (at 1230.73 183.78) (size 0.6) (drill 0.3) (layers "F.Cu" "B.Cu") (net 18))
 (segment (start 1288.74 25.05) (end 1288.74 29.1) (width 0.25) (layer "F.Cu") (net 18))
 (segment (start 1288.74 29.1) (end 1288.74 183.78) (width 0.25) (layer "F.Cu") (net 18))
 (via (at 1288.74 183.78) (size 0.6) (drill 0.3) (layers "F.Cu" "B.Cu") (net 18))
 (segment (start 1230.73 183.78) (end 1288.74 183.78) (width 0.25) (layer "B.Cu") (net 18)))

